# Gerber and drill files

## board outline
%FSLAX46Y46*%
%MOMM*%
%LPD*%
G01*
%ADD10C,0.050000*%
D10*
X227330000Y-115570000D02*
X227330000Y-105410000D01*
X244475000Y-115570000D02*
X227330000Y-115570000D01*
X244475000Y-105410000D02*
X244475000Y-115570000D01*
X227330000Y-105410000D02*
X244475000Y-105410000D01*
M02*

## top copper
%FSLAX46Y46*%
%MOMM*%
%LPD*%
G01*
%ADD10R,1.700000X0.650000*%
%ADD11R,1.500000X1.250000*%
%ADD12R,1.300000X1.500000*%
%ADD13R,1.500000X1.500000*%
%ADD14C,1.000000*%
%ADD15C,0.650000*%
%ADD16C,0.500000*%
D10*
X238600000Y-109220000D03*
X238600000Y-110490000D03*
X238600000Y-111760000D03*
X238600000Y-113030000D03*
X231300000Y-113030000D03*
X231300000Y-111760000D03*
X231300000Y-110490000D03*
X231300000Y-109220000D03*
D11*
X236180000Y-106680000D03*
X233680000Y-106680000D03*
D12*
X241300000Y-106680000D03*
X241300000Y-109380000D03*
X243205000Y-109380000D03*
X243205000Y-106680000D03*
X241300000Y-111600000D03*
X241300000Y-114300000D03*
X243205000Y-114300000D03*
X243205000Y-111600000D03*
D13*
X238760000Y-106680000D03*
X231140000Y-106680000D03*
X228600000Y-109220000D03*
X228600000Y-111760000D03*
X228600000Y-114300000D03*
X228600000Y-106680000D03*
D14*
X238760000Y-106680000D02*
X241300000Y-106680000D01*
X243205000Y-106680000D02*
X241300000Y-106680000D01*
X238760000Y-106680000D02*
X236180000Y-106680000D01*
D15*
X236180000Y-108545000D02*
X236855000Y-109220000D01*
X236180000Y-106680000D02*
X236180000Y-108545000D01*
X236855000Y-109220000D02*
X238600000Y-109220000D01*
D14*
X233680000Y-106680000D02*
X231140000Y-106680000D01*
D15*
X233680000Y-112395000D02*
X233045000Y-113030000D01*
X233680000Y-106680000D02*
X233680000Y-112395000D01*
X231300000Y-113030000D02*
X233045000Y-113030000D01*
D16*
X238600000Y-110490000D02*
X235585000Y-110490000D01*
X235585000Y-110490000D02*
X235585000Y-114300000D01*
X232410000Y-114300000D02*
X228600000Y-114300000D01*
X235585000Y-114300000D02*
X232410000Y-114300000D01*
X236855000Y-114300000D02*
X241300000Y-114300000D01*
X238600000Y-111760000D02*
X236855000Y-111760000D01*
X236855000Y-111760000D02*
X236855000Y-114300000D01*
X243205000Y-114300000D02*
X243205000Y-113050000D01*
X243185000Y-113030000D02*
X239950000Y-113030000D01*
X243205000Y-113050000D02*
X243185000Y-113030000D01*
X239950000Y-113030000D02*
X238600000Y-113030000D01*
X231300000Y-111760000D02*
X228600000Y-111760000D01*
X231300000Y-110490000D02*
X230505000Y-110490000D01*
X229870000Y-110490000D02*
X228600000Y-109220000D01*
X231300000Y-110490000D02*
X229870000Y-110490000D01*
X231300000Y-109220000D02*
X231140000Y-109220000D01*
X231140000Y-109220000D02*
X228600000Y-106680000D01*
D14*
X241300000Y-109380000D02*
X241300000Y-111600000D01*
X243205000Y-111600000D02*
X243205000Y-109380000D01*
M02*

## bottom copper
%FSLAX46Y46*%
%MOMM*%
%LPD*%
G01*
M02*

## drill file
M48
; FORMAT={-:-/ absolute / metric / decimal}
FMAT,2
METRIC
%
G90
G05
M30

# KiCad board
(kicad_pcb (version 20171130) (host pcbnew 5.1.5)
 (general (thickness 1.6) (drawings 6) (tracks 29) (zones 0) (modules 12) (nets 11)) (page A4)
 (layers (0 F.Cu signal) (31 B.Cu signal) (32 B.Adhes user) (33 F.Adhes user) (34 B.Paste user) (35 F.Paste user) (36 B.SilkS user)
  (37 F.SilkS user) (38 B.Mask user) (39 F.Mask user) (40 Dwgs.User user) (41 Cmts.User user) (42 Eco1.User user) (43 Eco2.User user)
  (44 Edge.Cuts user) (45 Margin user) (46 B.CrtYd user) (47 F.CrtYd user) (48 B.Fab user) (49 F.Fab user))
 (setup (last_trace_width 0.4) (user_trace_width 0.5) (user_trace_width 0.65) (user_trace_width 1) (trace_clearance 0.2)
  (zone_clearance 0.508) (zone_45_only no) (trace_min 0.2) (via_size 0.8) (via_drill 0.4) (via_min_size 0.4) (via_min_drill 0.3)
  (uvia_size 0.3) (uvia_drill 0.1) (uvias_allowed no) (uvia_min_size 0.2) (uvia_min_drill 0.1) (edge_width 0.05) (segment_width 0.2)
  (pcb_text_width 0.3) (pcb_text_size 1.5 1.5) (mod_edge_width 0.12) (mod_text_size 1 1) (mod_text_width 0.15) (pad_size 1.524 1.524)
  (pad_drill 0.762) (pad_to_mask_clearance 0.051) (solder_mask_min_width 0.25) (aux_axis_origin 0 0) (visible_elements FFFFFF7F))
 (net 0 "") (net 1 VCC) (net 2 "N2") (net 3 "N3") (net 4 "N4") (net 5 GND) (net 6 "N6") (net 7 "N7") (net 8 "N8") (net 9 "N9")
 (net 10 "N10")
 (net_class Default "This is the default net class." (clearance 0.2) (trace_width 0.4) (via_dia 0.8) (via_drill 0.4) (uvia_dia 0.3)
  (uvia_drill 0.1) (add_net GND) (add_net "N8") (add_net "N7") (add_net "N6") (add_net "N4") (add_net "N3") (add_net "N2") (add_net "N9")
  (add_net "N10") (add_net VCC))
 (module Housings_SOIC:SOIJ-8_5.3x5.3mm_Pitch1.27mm (layer F.Cu) (at 234.95 111.125)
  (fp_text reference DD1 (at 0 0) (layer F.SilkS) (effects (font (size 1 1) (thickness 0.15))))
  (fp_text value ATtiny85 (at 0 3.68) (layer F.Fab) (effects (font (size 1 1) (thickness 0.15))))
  (pad 8 smd rect (at 3.65 -1.905) (size 1.7 0.65) (layers F.Cu F.Paste F.Mask) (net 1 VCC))
  (pad 7 smd rect (at 3.65 -0.635) (size 1.7 0.65) (layers F.Cu F.Paste F.Mask) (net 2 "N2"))
  (pad 6 smd rect (at 3.65 0.635) (size 1.7 0.65) (layers F.Cu F.Paste F.Mask) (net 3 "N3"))
  (pad 5 smd rect (at 3.65 1.905) (size 1.7 0.65) (layers F.Cu F.Paste F.Mask) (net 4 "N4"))
  (pad 4 smd rect (at -3.65 1.905) (size 1.7 0.65) (layers F.Cu F.Paste F.Mask) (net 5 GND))
  (pad 3 smd rect (at -3.65 0.635) (size 1.7 0.65) (layers F.Cu F.Paste F.Mask) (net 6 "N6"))
  (pad 2 smd rect (at -3.65 -0.635) (size 1.7 0.65) (layers F.Cu F.Paste F.Mask) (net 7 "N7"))
  (pad 1 smd rect (at -3.65 -1.905) (size 1.7 0.65) (layers F.Cu F.Paste F.Mask) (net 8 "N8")))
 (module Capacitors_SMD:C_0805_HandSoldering (layer F.Cu) (at 234.93 106.68)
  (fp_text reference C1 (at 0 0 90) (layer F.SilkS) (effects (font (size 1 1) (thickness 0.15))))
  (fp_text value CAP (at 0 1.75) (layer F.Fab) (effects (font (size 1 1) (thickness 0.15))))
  (pad 2 smd rect (at 1.25 0) (size 1.5 1.25) (layers F.Cu F.Paste F.Mask) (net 1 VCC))
  (pad 1 smd rect (at -1.25 0) (size 1.5 1.25) (layers F.Cu F.Paste F.Mask) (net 5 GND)))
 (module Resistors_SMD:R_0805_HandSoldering (layer F.Cu) (at 241.3 108.03 90)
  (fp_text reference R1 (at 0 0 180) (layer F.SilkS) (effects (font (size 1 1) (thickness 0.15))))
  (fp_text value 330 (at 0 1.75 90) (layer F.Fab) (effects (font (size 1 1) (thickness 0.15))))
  (pad 2 smd rect (at 1.35 0 90) (size 1.5 1.3) (layers F.Cu F.Paste F.Mask) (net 1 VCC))
  (pad 1 smd rect (at -1.35 0 90) (size 1.5 1.3) (layers F.Cu F.Paste F.Mask) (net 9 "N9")))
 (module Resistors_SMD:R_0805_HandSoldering (layer F.Cu) (at 243.205 108.03 90)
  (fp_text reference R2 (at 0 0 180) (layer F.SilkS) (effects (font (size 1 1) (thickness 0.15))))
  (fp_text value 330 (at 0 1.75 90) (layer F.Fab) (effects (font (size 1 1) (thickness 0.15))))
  (pad 1 smd rect (at -1.35 0 90) (size 1.5 1.3) (layers F.Cu F.Paste F.Mask) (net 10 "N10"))
  (pad 2 smd rect (at 1.35 0 90) (size 1.5 1.3) (layers F.Cu F.Paste F.Mask) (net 1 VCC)))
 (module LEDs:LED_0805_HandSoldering (layer F.Cu) (at 241.3 112.95 90)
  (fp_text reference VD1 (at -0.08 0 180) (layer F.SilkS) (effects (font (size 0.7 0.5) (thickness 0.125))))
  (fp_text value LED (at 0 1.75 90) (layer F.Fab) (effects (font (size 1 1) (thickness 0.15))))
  (pad 2 smd rect (at 1.35 0 90) (size 1.5 1.3) (layers F.Cu F.Paste F.Mask) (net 9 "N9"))
  (pad 1 smd rect (at -1.35 0 90) (size 1.5 1.3) (layers F.Cu F.Paste F.Mask) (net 3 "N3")))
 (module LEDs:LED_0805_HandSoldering (layer F.Cu) (at 243.205 112.95 90)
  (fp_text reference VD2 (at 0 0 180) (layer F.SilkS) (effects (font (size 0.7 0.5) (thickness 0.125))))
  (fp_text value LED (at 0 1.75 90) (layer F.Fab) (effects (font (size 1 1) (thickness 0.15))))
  (pad 1 smd rect (at -1.35 0 90) (size 1.5 1.3) (layers F.Cu F.Paste F.Mask) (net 4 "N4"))
  (pad 2 smd rect (at 1.35 0 90) (size 1.5 1.3) (layers F.Cu F.Paste F.Mask) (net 10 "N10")))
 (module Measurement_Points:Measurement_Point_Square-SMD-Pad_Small (layer F.Cu) (at 238.76 106.68 180)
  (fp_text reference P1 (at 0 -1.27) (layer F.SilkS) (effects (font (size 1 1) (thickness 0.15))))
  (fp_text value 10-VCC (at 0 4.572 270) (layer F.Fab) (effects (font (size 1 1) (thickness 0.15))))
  (pad 1 smd rect (at 0 0 180) (size 1.5 1.5) (layers F.Cu F.Mask) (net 1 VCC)))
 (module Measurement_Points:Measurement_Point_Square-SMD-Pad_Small (layer F.Cu) (at 231.14 106.68 180)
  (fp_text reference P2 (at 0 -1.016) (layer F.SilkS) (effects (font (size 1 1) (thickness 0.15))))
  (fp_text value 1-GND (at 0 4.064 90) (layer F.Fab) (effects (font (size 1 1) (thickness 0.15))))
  (pad 1 smd rect (at 0 0 180) (size 1.5 1.5) (layers F.Cu F.Mask) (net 5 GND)))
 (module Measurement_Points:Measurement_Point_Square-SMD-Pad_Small (layer F.Cu) (at 228.6 109.22 180)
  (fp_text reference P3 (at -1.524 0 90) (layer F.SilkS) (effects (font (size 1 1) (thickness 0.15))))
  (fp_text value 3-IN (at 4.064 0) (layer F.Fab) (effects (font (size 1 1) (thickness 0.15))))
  (pad 1 smd rect (at 0 0 180) (size 1.5 1.5) (layers F.Cu F.Mask) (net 7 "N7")))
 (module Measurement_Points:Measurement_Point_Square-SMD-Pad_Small (layer F.Cu) (at 228.6 111.76 180)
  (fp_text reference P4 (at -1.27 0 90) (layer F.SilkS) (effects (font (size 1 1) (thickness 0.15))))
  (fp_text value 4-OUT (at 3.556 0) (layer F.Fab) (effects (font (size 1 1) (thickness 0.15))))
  (pad 1 smd rect (at 0 0 180) (size 1.5 1.5) (layers F.Cu F.Mask) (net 6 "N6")))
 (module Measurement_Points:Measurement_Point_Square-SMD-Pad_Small (layer F.Cu) (at 228.6 114.3 180)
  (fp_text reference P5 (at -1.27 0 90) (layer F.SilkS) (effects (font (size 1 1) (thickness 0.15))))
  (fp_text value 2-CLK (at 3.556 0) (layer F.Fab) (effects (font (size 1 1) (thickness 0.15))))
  (pad 1 smd rect (at 0 0 180) (size 1.5 1.5) (layers F.Cu F.Mask) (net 2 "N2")))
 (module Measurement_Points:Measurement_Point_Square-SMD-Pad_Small (layer F.Cu) (at 228.6 106.68 180)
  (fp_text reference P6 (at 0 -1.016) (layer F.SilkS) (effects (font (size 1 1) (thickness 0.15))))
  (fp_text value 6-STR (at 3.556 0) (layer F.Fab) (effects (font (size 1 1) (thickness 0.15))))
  (pad 1 smd rect (at 0 0 180) (size 1.5 1.5) (layers F.Cu F.Mask) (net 8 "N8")))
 (gr_line (start 227.33 115.57) (end 227.33 105.41) (layer Edge.Cuts) (width 0.05))
 (gr_line (start 244.475 115.57) (end 227.33 115.57) (layer Edge.Cuts) (width 0.05))
 (gr_line (start 244.475 105.41) (end 244.475 115.57) (layer Edge.Cuts) (width 0.05))
 (gr_line (start 227.33 105.41) (end 244.475 105.41) (layer Edge.Cuts) (width 0.05))
 (segment (start 238.76 106.68) (end 241.3 106.68) (width 1) (layer F.Cu) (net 1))
 (segment (start 243.205 106.68) (end 241.3 106.68) (width 1) (layer F.Cu) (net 1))
 (segment (start 238.76 106.68) (end 236.18 106.68) (width 1) (layer F.Cu) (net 1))
 (segment (start 236.18 108.545) (end 236.855 109.22) (width 0.65) (layer F.Cu) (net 1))
 (segment (start 236.18 106.68) (end 236.18 108.545) (width 0.65) (layer F.Cu) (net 1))
 (segment (start 236.855 109.22) (end 238.6 109.22) (width 0.65) (layer F.Cu) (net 1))
 (segment (start 233.68 106.68) (end 231.14 106.68) (width 1) (layer F.Cu) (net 5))
 (segment (start 233.68 112.395) (end 233.045 113.03) (width 0.65) (layer F.Cu) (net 5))
 (segment (start 233.68 106.68) (end 233.68 112.395) (width 0.65) (layer F.Cu) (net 5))
 (segment (start 231.3 113.03) (end 233.045 113.03) (width 0.65) (layer F.Cu) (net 5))
 (segment (start 238.6 110.49) (end 235.585 110.49) (width 0.5) (layer F.Cu) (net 2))
 (segment (start 235.585 110.49) (end 235.585 114.3) (width 0.5) (layer F.Cu) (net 2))
 (segment (start 232.41 114.3) (end 228.6 114.3) (width 0.5) (layer F.Cu) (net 2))
 (segment (start 235.585 114.3) (end 232.41 114.3) (width 0.5) (layer F.Cu) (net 2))
 (segment (start 236.855 114.3) (end 241.3 114.3) (width 0.5) (layer F.Cu) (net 3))
 (segment (start 238.6 111.76) (end 236.855 111.76) (width 0.5) (layer F.Cu) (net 3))
 (segment (start 236.855 111.76) (end 236.855 114.3) (width 0.5) (layer F.Cu) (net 3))
 (segment (start 243.205 114.3) (end 243.205 113.05) (width 0.5) (layer F.Cu) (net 4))
 (segment (start 243.185 113.03) (end 239.95 113.03) (width 0.5) (layer F.Cu) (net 4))
 (segment (start 243.205 113.05) (end 243.185 113.03) (width 0.5) (layer F.Cu) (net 4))
 (segment (start 239.95 113.03) (end 238.6 113.03) (width 0.5) (layer F.Cu) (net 4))
 (segment (start 231.3 111.76) (end 228.6 111.76) (width 0.5) (layer F.Cu) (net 6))
 (segment (start 231.3 110.49) (end 230.505 110.49) (width 0.5) (layer F.Cu) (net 7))
 (segment (start 229.87 110.49) (end 228.6 109.22) (width 0.5) (layer F.Cu) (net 7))
 (segment (start 231.3 110.49) (end 229.87 110.49) (width 0.5) (layer F.Cu) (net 7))
 (segment (start 231.3 109.22) (end 231.14 109.22) (width 0.5) (layer F.Cu) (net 8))
 (segment (start 231.14 109.22) (end 228.6 106.68) (width 0.5) (layer F.Cu) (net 8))
 (segment (start 241.3 109.38) (end 241.3 111.6) (width 1) (layer F.Cu) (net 9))
 (segment (start 243.205 111.6) (end 243.205 109.38) (width 1) (layer F.Cu) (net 10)))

